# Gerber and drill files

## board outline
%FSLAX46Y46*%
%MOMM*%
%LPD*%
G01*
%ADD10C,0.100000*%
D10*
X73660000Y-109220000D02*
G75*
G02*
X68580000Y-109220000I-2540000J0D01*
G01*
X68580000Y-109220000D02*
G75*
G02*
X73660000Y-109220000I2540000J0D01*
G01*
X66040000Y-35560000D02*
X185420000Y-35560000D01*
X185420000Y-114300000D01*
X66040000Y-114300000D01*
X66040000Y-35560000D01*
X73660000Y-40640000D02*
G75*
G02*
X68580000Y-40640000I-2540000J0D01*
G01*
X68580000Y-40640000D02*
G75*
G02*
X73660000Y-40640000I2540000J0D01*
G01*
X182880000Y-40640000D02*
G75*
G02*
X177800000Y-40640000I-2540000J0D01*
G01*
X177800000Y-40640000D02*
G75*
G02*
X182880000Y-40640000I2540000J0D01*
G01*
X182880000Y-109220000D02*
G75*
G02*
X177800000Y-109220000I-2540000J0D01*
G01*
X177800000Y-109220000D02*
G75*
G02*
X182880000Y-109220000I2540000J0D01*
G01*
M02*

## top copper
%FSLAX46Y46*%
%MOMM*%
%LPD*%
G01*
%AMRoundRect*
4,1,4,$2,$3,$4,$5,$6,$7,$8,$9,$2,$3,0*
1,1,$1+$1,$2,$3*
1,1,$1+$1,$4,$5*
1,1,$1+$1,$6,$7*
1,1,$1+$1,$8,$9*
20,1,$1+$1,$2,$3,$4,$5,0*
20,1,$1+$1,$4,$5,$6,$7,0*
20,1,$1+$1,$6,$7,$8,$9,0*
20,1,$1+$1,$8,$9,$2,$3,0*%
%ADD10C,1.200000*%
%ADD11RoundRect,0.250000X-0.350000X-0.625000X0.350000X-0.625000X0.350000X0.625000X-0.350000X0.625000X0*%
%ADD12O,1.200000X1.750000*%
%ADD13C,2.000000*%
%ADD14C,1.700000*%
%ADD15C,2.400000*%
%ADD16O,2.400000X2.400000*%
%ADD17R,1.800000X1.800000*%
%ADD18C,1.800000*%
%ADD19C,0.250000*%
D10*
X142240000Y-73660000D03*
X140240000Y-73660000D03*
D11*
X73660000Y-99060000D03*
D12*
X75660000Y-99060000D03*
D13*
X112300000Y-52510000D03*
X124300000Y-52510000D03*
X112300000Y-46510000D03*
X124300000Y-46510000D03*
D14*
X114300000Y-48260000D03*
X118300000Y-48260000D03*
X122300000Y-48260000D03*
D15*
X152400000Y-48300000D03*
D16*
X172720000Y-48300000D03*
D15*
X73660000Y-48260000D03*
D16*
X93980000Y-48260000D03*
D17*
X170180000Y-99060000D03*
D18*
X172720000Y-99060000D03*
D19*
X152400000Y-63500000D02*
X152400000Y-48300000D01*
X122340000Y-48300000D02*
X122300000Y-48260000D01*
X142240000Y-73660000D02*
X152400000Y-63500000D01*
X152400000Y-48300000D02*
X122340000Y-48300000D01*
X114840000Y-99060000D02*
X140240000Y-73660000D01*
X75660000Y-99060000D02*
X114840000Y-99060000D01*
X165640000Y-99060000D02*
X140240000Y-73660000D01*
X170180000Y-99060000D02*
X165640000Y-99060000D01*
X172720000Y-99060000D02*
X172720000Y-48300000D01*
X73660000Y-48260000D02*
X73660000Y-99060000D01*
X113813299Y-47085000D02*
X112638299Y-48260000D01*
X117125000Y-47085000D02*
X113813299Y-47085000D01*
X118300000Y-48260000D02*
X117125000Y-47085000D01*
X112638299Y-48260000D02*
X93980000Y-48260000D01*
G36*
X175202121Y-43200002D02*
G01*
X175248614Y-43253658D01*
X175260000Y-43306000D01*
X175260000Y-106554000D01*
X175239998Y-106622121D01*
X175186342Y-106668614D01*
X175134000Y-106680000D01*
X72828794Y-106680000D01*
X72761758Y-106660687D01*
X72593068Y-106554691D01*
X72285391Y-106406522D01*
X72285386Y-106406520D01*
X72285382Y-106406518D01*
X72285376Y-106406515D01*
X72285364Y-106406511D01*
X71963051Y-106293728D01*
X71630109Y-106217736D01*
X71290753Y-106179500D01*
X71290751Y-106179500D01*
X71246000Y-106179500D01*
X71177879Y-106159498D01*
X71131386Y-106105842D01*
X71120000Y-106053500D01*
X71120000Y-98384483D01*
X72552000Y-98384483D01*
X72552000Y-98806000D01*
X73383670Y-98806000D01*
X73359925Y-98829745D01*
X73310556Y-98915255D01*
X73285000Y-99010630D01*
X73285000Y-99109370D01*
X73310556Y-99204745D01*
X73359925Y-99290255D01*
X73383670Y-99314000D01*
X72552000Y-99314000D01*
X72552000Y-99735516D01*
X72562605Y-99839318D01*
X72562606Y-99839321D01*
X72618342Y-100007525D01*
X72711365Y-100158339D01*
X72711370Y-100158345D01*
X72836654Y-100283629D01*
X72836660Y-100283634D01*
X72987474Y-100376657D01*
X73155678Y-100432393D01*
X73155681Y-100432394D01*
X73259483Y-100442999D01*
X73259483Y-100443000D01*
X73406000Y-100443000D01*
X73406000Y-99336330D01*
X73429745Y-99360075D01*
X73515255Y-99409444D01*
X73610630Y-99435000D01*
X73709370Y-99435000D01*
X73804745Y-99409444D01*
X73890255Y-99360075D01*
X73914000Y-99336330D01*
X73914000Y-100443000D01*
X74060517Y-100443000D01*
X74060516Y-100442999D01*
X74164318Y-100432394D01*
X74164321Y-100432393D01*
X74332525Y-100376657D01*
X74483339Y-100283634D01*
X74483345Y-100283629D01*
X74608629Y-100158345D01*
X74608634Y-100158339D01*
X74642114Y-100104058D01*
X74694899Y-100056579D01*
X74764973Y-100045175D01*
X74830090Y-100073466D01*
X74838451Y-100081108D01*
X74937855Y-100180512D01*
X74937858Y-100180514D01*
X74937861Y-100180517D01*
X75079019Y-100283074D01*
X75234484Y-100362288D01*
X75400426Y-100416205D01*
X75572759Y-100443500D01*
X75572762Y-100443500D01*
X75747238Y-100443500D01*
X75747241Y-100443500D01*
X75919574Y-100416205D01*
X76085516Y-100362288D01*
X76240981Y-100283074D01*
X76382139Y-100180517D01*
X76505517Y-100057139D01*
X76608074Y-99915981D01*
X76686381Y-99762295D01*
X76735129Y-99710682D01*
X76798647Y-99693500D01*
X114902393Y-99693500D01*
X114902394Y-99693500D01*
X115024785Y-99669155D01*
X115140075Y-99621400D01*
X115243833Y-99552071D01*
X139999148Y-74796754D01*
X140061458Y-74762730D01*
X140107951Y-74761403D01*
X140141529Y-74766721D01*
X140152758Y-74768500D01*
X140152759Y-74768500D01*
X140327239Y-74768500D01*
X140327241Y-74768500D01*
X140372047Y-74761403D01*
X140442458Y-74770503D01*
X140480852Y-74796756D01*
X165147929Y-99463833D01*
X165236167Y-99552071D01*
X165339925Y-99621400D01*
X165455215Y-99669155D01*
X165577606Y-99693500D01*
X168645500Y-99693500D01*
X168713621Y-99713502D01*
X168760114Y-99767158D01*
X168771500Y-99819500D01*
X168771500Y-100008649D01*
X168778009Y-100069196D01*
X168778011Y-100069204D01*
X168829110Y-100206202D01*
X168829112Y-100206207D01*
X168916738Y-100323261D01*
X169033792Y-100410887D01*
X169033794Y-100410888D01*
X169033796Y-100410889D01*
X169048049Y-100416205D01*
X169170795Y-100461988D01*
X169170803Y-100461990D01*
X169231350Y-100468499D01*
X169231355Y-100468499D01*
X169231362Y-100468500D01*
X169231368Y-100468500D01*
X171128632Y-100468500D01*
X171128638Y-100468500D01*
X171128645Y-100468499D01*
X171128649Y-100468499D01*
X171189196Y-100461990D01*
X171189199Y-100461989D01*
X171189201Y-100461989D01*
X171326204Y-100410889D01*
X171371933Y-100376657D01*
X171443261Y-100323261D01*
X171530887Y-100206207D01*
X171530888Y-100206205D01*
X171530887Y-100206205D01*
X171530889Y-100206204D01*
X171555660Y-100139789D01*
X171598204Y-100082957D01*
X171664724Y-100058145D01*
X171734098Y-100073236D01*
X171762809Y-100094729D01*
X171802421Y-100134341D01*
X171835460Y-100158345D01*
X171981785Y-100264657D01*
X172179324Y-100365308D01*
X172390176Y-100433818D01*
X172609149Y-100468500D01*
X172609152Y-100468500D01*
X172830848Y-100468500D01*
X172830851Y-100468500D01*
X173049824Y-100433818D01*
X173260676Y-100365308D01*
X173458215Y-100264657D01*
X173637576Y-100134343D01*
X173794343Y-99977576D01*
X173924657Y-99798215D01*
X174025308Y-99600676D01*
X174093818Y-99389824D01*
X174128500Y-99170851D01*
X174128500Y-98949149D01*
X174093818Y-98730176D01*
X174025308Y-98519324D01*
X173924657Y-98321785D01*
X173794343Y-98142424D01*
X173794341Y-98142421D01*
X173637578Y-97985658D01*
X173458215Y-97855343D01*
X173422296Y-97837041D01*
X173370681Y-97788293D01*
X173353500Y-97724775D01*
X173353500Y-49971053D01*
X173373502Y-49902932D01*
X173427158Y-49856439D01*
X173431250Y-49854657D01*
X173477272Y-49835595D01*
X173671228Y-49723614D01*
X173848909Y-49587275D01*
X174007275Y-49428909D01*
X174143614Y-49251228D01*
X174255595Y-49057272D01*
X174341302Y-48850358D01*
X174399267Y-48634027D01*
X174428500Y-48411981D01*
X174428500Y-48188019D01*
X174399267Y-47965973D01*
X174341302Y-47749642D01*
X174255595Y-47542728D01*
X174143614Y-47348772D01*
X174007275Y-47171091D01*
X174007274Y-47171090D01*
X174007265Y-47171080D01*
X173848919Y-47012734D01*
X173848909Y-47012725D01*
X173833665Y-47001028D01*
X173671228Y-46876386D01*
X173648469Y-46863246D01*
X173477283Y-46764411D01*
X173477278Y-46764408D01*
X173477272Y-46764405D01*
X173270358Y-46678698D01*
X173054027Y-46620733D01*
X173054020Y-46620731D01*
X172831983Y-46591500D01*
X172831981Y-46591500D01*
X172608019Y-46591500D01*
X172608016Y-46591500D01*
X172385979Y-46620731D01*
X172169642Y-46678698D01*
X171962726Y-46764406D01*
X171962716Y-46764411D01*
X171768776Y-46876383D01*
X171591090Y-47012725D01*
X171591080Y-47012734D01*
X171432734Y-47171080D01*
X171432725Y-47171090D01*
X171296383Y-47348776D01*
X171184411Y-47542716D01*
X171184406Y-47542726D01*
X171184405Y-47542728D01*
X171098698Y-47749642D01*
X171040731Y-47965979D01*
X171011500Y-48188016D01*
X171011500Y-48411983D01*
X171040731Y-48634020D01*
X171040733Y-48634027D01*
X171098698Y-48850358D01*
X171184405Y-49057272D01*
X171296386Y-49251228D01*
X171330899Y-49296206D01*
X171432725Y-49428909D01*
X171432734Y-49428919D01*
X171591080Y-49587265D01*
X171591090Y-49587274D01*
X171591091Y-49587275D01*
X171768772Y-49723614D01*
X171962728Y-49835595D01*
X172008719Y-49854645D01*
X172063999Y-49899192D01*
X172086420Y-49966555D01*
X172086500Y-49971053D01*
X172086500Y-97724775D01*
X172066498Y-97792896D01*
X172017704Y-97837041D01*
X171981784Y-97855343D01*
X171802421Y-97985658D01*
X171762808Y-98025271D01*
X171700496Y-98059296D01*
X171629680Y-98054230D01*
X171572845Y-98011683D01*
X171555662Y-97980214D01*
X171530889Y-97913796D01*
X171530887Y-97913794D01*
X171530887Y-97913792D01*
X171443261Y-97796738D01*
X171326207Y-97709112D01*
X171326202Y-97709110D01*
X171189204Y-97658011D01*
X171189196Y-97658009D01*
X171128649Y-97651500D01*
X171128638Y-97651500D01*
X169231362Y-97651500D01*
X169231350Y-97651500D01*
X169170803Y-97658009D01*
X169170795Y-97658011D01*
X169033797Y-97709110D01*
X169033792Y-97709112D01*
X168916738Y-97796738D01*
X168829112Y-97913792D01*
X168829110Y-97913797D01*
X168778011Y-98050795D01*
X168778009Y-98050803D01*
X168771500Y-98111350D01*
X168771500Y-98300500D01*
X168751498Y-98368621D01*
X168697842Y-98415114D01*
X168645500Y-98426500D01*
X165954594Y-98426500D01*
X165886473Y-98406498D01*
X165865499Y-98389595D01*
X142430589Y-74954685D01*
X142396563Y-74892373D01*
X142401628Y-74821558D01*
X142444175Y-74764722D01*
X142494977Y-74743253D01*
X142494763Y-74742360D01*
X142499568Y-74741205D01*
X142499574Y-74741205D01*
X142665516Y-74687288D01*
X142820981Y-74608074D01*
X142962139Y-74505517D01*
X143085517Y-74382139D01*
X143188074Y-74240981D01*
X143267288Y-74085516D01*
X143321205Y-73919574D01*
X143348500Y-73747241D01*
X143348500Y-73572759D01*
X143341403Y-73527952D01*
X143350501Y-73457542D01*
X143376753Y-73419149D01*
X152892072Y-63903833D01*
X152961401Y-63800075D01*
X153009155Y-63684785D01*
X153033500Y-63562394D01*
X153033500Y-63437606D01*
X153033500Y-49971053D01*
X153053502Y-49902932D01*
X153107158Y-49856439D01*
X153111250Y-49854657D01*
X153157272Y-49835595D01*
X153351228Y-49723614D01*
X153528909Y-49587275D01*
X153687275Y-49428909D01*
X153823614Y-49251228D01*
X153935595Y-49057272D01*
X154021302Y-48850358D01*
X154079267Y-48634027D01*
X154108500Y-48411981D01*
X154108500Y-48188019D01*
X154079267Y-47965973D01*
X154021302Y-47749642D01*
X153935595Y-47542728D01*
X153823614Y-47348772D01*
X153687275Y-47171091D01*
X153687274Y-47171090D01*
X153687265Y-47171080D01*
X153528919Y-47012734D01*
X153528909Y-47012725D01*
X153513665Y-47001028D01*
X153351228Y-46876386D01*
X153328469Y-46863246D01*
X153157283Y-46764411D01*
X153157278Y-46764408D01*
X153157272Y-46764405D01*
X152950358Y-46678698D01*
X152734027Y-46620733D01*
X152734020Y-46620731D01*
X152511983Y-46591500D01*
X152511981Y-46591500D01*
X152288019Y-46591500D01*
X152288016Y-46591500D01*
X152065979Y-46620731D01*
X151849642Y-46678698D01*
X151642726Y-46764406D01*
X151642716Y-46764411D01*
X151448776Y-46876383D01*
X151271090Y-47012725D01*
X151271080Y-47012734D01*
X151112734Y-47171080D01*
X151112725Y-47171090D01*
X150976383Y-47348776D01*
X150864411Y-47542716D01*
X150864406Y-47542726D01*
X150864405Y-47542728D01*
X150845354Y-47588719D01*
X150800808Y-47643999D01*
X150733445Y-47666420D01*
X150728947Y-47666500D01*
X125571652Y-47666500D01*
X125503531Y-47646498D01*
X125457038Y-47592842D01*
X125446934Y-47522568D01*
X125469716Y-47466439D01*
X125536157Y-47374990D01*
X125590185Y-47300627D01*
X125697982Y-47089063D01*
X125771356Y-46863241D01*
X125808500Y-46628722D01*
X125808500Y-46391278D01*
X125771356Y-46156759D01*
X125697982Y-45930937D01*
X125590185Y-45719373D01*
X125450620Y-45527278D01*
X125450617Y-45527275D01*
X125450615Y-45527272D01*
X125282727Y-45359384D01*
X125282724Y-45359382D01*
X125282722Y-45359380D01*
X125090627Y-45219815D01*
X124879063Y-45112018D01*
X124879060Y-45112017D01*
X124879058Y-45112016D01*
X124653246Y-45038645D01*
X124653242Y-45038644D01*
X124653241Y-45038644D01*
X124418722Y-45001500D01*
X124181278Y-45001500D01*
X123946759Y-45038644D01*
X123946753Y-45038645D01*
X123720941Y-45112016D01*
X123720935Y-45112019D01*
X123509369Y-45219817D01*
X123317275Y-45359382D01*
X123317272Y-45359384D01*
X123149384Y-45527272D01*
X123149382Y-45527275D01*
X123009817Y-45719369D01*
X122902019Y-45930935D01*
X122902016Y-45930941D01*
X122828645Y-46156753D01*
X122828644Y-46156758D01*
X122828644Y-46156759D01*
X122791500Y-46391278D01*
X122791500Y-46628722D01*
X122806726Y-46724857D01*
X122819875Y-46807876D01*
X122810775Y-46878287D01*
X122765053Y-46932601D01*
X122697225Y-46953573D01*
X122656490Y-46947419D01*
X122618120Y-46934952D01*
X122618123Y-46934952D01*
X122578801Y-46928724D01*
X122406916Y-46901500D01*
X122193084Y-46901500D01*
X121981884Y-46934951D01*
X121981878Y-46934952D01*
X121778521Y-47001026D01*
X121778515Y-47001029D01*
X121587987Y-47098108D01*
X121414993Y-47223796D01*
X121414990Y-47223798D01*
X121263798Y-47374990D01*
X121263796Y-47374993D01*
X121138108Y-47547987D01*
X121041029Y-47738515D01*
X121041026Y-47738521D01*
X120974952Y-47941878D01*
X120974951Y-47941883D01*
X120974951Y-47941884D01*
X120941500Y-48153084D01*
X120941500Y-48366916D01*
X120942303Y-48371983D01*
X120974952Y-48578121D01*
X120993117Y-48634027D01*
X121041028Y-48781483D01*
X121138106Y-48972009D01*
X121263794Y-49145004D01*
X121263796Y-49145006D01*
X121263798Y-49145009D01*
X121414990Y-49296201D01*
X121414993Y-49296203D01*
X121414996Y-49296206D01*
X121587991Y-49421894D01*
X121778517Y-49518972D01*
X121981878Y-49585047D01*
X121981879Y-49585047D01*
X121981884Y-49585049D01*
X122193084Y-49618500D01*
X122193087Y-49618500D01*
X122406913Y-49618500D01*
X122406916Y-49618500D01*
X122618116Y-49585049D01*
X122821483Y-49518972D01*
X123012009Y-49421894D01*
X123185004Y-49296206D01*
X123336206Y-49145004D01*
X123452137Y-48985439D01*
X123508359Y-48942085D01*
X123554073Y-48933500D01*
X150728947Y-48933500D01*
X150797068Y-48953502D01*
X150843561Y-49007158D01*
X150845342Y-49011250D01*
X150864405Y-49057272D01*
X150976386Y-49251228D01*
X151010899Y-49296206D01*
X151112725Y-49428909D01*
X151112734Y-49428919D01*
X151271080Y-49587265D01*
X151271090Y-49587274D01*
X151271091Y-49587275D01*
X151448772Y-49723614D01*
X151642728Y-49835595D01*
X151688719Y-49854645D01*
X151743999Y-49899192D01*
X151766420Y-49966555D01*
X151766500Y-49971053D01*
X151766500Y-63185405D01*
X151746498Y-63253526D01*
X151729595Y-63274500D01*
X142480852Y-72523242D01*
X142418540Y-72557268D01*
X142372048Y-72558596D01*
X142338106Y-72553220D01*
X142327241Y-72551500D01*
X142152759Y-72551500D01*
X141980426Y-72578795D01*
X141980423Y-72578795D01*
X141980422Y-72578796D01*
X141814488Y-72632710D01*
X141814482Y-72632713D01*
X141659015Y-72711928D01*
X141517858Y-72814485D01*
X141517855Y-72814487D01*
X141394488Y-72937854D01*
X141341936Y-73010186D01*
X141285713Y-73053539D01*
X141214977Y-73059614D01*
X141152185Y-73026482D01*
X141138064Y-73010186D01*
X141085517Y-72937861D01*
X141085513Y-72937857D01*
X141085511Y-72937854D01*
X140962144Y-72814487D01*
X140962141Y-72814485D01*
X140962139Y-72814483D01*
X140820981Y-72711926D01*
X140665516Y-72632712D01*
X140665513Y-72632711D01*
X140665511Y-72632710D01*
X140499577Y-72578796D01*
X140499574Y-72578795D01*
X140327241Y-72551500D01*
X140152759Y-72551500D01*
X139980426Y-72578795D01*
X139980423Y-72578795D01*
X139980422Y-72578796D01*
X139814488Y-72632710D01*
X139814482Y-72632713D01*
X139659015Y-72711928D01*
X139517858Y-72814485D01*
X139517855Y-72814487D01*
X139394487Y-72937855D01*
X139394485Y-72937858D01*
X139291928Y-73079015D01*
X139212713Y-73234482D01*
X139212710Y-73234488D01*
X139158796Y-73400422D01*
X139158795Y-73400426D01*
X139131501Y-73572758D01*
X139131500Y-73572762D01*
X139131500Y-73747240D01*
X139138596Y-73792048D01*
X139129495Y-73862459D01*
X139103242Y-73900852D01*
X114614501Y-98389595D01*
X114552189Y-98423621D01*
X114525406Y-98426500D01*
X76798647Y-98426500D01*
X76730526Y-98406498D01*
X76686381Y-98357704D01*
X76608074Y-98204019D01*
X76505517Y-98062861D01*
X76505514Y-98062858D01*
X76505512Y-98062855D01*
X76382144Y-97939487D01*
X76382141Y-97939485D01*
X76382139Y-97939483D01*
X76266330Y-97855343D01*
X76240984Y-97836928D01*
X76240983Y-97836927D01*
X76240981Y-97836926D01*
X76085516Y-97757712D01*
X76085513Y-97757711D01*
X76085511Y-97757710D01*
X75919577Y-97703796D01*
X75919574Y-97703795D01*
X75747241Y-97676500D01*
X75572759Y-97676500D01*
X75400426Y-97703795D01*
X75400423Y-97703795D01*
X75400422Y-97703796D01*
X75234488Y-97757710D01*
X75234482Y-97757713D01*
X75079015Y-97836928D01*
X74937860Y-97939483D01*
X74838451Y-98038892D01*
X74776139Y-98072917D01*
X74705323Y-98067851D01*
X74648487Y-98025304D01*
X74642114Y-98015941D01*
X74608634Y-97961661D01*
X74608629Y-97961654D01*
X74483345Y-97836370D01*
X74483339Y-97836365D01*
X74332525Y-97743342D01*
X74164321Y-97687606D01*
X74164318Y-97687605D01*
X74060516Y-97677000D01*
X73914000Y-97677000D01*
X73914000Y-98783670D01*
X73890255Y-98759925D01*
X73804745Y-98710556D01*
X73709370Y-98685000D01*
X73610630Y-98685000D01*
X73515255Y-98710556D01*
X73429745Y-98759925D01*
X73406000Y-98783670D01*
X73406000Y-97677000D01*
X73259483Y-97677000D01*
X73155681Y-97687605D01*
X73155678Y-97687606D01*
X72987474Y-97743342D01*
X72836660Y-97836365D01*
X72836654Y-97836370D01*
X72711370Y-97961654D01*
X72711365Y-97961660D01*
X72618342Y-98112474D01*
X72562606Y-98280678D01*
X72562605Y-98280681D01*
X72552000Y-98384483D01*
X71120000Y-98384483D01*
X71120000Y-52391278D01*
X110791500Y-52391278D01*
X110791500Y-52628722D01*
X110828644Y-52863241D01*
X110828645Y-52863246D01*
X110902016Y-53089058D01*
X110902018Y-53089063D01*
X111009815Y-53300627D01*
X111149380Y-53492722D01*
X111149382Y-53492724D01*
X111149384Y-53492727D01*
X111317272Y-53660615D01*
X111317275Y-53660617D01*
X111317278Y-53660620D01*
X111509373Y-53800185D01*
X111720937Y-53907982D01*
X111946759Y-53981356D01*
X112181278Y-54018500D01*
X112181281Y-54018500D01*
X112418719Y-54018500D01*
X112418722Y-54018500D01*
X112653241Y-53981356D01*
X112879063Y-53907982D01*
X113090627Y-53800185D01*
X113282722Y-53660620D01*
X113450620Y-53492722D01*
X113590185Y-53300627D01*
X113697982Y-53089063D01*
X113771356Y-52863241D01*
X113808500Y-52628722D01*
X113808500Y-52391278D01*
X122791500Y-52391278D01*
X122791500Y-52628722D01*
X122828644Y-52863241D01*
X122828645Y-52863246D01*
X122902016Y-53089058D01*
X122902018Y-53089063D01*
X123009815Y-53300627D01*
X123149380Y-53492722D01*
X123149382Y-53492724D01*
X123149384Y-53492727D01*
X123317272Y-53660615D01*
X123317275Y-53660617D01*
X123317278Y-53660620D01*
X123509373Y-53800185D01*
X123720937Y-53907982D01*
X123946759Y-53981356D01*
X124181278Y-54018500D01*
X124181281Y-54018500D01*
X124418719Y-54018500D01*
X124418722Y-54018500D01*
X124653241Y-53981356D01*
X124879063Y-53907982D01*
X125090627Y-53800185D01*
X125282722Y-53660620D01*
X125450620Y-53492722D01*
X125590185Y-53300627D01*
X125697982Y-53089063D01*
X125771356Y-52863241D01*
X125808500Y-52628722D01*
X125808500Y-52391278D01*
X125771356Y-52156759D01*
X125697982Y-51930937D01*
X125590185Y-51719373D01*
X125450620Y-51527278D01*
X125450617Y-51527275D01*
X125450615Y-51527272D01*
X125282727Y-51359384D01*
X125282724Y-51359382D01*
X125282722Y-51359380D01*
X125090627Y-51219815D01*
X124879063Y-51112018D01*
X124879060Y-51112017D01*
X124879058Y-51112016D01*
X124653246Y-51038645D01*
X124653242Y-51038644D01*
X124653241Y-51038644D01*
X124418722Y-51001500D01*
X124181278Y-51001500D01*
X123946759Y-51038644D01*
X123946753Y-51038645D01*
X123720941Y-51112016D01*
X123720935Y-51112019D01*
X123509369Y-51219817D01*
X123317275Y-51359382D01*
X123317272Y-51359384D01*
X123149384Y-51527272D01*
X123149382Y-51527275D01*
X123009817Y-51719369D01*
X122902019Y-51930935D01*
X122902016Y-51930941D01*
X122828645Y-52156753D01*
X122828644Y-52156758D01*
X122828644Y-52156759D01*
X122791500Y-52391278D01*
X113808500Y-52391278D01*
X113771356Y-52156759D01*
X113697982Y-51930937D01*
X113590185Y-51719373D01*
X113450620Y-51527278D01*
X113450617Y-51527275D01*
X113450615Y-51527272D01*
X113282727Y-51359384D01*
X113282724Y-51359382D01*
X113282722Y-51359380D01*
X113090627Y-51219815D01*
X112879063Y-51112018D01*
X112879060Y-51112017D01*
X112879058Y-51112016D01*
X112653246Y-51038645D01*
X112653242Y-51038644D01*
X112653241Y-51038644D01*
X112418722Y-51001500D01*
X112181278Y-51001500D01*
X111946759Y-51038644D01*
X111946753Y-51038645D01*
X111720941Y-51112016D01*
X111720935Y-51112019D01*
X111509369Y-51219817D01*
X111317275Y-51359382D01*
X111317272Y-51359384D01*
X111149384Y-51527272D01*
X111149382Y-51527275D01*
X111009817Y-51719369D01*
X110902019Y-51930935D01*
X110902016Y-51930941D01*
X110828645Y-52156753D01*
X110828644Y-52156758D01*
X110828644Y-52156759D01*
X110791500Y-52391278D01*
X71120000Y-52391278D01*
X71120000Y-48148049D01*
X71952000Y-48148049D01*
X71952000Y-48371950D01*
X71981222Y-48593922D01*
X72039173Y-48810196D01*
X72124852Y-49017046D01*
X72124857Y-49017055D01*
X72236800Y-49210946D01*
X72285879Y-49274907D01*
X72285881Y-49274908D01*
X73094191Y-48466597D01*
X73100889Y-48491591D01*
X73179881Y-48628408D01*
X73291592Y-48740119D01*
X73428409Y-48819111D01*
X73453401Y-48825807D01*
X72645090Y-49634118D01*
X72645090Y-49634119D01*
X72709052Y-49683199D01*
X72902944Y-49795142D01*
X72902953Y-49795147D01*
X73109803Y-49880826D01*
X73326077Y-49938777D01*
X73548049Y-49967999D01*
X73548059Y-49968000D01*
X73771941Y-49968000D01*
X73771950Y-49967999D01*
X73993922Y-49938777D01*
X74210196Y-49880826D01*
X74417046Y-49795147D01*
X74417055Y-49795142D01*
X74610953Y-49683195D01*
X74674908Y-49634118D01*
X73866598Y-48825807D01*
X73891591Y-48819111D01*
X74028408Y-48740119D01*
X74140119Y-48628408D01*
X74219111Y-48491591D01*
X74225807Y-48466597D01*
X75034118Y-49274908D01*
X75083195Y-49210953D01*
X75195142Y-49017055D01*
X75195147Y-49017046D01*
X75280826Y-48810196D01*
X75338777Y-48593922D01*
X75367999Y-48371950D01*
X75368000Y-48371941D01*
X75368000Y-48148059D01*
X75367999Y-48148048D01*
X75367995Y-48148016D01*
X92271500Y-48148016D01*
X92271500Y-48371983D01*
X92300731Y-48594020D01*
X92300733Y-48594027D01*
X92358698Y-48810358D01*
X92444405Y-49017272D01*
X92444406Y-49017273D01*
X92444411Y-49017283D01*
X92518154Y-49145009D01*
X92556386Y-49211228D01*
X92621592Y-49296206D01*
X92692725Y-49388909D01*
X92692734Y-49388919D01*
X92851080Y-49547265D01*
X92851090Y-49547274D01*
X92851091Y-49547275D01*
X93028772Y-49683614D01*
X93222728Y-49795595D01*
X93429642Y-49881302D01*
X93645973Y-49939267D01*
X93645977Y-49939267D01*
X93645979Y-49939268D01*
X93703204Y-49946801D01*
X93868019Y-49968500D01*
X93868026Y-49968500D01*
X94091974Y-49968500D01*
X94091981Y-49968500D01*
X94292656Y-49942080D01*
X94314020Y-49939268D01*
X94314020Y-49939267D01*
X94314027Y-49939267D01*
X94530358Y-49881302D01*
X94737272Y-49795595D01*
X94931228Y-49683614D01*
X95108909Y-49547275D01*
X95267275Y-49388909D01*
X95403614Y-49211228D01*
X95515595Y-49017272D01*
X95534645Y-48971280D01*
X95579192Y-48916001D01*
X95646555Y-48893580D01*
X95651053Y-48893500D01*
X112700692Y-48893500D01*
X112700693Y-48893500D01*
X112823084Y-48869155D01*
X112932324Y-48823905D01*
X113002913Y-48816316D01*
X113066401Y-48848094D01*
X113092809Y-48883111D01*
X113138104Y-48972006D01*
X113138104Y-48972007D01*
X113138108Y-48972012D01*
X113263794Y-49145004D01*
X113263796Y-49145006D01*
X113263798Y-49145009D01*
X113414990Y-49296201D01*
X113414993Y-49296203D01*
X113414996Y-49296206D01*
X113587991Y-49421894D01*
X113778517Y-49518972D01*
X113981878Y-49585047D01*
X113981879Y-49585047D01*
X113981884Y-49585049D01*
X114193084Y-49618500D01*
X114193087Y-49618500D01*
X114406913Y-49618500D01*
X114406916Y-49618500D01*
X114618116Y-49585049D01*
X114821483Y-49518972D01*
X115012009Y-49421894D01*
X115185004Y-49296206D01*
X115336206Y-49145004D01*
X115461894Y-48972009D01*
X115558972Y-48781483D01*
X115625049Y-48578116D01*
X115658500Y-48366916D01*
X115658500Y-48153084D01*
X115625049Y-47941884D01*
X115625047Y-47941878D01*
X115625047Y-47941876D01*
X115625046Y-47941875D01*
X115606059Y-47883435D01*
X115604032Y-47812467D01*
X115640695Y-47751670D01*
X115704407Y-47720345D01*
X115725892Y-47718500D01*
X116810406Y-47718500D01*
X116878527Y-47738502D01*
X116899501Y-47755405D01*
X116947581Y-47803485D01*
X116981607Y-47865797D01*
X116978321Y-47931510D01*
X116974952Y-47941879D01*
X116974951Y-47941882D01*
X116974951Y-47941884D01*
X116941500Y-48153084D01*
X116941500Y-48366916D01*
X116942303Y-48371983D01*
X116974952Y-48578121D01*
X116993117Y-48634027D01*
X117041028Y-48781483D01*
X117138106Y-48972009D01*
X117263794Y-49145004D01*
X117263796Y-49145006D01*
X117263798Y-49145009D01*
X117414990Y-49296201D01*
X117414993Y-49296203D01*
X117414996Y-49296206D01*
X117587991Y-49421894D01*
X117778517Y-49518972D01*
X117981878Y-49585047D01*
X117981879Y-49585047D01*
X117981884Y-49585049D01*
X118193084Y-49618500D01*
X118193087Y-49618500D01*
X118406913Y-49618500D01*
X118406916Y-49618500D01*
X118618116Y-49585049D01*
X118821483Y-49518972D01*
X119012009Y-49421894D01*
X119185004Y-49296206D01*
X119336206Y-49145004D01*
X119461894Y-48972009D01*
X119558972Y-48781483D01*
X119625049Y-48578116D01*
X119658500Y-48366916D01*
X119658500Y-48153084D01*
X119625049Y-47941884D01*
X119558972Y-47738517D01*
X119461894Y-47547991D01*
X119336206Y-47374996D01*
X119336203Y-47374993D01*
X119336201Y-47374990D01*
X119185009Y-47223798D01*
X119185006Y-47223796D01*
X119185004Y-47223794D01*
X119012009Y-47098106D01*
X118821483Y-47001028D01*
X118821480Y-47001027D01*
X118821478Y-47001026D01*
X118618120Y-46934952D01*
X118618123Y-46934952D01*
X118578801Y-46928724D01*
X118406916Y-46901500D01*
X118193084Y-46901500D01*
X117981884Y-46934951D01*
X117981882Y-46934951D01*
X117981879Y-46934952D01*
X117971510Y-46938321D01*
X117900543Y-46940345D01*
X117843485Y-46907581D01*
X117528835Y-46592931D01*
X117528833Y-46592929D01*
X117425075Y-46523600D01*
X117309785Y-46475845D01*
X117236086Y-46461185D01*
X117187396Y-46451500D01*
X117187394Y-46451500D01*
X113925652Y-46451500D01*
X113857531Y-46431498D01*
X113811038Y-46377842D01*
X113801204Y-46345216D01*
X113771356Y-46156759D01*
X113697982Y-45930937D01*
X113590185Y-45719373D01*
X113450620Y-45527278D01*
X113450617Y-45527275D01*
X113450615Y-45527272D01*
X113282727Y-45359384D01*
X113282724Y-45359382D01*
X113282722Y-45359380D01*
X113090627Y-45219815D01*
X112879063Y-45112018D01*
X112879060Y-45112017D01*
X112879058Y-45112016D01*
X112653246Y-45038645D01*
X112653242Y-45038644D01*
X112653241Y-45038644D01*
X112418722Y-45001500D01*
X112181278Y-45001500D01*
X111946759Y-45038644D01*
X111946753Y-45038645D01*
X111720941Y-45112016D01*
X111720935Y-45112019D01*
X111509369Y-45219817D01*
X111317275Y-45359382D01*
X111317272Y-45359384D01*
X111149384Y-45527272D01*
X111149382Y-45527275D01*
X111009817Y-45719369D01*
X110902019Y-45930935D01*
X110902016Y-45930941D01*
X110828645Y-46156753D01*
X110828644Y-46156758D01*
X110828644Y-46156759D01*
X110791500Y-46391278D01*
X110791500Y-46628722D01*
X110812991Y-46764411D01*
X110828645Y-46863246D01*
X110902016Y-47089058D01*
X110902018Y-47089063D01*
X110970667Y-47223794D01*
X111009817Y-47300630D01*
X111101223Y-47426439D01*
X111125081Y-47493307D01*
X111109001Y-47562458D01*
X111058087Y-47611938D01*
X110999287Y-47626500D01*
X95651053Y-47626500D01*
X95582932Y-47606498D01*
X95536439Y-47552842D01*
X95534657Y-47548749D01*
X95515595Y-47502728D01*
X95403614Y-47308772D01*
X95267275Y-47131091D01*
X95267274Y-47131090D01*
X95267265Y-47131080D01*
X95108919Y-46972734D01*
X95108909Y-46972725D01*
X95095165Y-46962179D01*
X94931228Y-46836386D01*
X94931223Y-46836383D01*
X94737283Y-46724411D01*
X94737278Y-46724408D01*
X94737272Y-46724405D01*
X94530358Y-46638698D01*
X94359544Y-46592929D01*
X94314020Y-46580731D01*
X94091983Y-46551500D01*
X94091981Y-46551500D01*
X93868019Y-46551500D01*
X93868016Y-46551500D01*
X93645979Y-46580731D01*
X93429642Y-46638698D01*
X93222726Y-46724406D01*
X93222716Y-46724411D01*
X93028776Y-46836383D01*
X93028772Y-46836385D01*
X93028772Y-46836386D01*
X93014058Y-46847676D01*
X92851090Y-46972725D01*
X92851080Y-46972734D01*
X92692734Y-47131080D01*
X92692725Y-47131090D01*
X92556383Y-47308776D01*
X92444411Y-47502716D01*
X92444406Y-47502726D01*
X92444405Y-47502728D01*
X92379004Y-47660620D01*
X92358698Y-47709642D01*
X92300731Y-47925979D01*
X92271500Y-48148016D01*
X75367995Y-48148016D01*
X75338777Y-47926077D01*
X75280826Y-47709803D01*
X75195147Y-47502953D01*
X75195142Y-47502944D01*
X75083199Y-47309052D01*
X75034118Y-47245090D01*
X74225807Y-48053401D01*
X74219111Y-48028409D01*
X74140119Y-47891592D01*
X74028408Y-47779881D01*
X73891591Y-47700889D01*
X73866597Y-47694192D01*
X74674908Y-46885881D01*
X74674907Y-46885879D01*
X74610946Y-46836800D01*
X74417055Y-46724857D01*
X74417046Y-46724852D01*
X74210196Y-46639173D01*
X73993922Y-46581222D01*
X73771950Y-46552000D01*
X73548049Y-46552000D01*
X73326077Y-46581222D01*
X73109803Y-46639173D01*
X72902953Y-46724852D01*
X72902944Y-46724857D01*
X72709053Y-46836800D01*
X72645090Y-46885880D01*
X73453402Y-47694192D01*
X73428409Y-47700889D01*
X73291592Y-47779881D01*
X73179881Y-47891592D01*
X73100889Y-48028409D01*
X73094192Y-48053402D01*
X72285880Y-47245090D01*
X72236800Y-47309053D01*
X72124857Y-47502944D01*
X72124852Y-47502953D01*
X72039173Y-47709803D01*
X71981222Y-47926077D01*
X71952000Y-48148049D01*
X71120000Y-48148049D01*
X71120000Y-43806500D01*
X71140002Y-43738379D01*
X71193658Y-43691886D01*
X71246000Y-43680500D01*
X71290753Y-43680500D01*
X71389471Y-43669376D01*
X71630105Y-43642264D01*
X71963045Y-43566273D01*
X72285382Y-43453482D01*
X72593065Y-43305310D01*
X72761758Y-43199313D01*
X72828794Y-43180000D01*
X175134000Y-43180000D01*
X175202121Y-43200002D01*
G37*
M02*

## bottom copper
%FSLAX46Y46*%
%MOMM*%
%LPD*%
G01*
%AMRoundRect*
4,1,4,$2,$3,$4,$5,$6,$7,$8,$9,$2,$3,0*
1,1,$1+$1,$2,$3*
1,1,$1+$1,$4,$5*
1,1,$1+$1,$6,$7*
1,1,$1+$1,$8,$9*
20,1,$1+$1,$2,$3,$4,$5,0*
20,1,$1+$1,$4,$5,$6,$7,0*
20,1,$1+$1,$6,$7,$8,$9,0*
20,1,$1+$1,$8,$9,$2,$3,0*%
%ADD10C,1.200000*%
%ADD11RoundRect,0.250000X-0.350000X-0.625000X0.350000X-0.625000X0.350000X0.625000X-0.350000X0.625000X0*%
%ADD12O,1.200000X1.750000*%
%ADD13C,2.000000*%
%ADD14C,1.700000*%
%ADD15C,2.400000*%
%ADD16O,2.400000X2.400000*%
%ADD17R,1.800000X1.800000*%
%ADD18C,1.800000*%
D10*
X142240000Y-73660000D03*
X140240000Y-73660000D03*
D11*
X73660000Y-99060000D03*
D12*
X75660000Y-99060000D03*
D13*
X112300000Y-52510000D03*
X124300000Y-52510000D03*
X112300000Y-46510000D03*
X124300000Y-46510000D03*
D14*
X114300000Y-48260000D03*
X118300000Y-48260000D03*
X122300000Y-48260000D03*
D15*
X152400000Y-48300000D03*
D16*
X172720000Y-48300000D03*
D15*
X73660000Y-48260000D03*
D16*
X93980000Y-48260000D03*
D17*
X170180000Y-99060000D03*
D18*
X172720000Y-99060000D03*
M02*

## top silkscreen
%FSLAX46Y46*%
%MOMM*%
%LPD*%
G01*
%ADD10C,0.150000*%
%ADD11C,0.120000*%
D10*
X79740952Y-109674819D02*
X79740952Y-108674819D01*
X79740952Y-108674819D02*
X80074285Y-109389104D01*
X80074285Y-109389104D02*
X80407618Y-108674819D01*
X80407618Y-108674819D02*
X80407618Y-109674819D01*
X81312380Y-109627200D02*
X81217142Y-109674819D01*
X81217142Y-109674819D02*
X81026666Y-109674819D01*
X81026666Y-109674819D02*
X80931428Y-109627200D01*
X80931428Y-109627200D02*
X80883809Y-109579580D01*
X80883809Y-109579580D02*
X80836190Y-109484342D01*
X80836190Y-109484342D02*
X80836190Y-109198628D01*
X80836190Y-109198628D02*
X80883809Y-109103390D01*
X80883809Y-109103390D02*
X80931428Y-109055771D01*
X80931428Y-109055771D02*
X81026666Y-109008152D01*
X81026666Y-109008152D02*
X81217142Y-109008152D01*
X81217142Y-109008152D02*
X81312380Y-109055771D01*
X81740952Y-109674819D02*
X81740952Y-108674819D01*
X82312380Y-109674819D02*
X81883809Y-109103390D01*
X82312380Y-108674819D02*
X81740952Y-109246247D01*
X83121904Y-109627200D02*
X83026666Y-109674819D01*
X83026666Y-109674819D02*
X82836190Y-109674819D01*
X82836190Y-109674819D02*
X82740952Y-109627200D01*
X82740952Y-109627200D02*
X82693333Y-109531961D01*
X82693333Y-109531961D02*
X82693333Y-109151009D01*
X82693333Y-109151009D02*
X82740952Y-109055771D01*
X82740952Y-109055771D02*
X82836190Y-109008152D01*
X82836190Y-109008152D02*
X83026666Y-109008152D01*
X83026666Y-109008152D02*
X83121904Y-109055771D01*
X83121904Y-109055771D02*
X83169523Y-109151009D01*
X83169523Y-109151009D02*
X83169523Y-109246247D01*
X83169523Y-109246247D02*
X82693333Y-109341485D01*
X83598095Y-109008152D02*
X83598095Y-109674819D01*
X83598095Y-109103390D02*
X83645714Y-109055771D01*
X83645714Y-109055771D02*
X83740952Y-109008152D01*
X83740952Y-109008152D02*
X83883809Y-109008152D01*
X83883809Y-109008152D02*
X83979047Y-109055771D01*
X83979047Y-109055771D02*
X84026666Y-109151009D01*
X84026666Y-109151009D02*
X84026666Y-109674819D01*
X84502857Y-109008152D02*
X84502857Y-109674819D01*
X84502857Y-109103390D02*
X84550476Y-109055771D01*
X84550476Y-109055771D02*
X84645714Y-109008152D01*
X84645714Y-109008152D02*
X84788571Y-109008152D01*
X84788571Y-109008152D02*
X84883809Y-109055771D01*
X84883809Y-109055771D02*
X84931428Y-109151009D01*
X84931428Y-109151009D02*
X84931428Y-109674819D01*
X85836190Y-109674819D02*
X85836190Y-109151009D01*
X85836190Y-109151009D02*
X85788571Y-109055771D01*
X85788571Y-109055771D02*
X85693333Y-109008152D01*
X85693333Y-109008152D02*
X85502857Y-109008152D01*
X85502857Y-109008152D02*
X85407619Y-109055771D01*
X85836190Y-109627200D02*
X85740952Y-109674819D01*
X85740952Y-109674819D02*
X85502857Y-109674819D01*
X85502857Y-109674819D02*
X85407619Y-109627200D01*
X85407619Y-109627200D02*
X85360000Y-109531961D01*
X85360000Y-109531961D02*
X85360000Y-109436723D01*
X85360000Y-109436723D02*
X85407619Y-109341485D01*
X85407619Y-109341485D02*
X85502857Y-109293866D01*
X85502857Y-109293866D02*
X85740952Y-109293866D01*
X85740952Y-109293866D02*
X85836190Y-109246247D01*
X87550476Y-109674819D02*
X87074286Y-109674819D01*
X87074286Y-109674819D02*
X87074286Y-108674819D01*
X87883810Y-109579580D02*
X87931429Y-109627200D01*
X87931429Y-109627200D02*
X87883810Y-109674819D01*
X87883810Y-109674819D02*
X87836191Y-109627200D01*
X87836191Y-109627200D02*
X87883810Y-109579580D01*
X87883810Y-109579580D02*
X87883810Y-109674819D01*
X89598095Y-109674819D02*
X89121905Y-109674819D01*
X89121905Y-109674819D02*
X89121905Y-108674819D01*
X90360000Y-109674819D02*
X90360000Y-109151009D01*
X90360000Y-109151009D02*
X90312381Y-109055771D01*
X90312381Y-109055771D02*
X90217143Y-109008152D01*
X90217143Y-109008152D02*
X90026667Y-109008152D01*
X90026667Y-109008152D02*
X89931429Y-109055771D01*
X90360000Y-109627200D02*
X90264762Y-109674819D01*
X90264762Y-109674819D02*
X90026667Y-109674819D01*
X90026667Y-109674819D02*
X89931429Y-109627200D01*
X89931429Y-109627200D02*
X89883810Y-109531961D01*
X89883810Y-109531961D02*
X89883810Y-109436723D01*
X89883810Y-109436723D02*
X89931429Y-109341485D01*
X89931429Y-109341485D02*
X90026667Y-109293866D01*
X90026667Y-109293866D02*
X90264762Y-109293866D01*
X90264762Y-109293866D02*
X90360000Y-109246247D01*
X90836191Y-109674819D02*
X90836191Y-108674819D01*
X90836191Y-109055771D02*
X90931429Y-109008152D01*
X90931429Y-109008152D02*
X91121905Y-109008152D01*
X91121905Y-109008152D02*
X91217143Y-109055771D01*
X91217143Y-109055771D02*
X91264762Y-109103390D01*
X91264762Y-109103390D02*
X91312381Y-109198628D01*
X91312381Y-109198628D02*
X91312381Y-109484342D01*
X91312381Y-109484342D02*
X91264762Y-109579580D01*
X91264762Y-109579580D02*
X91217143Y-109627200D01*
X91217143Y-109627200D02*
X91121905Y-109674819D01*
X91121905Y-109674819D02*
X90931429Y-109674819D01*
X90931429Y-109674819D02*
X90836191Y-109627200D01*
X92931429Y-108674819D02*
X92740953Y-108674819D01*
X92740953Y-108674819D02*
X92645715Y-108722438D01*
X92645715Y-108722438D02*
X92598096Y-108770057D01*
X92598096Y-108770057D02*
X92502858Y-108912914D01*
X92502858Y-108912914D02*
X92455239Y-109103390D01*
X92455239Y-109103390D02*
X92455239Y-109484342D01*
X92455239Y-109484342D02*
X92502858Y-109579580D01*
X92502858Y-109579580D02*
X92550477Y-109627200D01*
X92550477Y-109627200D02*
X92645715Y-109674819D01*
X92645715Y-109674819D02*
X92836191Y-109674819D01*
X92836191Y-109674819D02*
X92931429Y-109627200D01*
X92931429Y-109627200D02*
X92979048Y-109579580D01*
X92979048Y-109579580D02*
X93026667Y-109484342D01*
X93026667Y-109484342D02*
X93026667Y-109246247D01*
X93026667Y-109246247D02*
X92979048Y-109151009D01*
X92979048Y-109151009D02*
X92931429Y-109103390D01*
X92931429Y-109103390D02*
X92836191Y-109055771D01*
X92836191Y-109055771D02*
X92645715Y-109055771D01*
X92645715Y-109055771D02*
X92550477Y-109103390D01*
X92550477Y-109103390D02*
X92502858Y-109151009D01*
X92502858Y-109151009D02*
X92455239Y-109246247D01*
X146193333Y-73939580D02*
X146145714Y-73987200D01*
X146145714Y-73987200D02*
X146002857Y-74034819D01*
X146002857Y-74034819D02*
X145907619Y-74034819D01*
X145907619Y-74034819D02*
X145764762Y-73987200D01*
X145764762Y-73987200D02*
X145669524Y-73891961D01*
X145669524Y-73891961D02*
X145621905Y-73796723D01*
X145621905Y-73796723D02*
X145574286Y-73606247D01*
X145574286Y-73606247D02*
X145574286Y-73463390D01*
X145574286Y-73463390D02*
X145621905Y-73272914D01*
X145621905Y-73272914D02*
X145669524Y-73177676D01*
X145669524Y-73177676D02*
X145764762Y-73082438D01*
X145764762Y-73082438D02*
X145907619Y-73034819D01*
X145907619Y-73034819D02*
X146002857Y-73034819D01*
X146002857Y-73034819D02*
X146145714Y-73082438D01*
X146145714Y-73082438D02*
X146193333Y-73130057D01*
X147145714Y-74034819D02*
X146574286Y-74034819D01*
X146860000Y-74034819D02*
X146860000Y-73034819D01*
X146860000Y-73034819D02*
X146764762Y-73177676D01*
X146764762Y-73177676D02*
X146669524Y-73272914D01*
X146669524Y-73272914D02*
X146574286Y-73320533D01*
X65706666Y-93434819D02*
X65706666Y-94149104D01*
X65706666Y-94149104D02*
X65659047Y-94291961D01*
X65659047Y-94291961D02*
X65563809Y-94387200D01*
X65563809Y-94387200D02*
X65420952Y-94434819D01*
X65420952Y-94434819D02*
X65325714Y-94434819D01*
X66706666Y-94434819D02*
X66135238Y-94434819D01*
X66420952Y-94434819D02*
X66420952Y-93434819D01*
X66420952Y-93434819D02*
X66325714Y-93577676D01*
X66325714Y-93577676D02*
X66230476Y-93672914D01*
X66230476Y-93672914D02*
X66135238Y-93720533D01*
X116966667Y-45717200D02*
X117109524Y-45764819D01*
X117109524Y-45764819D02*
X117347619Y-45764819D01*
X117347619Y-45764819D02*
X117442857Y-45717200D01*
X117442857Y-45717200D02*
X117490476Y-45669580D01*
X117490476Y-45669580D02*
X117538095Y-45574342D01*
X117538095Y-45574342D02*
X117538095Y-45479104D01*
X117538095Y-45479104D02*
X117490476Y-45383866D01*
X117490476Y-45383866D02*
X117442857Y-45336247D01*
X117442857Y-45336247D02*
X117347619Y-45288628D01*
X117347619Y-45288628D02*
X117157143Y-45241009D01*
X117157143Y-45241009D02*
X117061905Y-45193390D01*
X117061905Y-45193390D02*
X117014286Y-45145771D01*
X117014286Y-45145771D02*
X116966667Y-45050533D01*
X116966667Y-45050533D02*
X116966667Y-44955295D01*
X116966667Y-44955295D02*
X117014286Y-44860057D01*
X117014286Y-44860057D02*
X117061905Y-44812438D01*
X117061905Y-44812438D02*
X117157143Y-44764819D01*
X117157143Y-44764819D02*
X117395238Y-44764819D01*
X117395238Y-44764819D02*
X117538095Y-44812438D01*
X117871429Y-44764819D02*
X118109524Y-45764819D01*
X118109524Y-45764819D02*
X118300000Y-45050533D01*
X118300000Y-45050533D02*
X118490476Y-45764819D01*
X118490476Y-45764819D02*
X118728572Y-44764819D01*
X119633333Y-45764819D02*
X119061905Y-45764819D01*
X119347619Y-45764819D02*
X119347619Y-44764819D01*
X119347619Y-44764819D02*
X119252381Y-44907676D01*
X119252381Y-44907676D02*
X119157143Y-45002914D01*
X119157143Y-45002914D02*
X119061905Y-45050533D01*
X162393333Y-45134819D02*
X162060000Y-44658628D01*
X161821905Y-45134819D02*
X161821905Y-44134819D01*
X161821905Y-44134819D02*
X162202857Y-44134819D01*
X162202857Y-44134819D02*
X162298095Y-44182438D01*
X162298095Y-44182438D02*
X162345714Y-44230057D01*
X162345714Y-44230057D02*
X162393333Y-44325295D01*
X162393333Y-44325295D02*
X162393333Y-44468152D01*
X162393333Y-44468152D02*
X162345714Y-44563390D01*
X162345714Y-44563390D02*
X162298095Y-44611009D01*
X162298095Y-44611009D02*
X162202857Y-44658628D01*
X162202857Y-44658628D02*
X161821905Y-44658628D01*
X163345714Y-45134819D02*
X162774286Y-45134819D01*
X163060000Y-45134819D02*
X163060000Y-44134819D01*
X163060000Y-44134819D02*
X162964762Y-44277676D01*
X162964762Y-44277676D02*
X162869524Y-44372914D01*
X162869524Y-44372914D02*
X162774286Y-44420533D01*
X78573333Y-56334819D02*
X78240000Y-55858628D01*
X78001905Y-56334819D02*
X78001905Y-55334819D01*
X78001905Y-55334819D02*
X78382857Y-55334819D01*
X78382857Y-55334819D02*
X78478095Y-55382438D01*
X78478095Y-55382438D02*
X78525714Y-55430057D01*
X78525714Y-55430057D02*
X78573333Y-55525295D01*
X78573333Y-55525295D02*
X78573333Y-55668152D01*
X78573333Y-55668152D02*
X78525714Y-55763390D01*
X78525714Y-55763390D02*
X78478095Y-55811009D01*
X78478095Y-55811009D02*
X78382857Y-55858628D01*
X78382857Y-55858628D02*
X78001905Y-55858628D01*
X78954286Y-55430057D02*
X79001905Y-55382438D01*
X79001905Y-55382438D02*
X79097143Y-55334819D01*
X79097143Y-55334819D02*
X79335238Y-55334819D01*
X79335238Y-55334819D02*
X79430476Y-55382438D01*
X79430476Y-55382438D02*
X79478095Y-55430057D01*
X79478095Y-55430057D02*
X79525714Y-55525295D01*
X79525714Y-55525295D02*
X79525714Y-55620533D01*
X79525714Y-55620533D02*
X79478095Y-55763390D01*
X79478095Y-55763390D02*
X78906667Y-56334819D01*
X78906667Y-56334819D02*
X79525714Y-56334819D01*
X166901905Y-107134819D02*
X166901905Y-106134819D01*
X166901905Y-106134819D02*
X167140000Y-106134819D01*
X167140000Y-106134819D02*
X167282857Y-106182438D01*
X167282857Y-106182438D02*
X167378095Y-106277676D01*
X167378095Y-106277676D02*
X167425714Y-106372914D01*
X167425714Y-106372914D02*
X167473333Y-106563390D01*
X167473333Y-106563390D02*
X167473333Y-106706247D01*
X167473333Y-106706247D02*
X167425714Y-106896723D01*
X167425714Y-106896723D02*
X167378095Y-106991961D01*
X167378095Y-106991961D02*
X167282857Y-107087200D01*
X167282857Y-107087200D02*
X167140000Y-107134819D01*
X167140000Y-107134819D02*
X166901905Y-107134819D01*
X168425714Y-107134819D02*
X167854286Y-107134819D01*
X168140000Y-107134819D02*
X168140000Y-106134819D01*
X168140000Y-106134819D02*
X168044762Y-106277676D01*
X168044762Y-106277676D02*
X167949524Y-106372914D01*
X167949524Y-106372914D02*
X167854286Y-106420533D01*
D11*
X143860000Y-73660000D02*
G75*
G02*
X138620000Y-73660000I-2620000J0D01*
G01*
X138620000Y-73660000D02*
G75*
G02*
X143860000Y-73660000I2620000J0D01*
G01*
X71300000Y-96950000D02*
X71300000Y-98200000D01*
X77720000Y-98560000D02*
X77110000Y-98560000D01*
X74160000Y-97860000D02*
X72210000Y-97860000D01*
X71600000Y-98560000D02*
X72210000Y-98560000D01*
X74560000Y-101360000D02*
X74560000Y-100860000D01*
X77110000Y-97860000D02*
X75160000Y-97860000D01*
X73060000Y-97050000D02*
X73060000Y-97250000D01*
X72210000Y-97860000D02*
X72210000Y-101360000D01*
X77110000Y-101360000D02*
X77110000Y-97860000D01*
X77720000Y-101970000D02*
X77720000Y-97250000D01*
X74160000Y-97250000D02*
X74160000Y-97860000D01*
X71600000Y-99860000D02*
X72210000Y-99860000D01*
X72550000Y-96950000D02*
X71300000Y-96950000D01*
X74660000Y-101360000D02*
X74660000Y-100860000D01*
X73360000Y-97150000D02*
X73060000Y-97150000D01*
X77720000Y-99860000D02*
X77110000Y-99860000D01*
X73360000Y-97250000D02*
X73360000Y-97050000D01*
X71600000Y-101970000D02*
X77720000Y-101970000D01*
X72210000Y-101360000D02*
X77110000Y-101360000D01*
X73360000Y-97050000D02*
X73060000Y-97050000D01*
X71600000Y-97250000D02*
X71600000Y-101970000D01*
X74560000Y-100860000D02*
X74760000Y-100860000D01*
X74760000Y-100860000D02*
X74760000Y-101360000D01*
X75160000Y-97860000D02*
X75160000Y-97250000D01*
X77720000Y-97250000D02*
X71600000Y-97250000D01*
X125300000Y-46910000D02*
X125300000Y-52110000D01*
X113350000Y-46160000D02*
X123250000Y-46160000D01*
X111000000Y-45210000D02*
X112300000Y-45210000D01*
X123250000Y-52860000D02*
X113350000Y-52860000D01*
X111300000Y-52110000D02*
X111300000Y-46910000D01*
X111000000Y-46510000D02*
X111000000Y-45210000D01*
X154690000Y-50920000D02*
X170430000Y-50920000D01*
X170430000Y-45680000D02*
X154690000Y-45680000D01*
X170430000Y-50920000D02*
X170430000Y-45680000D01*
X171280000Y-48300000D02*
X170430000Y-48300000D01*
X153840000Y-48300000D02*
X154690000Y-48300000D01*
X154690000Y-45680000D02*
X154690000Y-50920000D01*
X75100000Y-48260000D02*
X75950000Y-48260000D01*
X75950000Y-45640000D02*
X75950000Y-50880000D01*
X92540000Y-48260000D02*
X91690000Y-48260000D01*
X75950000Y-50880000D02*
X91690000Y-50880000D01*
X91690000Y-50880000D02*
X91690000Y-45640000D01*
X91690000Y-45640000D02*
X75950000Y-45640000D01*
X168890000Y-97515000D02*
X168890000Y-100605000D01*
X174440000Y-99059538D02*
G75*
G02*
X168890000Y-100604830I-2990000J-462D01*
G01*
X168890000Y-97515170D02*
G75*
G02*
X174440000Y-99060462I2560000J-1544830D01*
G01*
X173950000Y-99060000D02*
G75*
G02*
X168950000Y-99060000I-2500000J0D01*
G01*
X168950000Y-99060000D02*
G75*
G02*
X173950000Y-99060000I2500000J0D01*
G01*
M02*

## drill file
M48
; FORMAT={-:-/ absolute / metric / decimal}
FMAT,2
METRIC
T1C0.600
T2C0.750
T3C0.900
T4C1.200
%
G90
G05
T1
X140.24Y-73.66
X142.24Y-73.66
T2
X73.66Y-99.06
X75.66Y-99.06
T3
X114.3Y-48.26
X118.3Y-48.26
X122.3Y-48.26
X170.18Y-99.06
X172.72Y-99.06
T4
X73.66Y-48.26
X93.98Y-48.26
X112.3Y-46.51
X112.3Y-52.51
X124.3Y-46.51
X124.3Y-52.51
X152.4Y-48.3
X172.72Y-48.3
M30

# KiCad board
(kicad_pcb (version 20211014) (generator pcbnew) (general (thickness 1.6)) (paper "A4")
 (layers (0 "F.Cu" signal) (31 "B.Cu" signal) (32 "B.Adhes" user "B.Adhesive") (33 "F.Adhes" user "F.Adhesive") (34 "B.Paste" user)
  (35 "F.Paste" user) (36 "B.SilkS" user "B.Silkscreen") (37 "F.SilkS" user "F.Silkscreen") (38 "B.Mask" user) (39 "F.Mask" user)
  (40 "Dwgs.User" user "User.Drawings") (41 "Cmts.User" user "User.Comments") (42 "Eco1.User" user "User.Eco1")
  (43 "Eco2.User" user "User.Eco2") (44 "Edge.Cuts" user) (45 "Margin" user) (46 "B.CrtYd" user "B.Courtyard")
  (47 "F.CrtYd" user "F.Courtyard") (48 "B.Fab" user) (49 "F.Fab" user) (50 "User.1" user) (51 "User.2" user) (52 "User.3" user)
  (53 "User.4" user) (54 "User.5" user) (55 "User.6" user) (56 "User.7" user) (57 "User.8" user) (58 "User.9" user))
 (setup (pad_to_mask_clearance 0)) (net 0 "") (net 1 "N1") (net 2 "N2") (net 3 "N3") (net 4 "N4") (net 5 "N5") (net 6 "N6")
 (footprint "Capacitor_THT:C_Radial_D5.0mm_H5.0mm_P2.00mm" (layer "F.Cu") (at 142.24 73.66 180)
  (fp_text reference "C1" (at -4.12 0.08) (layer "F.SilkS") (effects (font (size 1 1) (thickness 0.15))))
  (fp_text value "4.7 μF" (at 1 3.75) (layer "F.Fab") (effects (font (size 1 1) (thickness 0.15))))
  (fp_circle (center 1 0) (end 3.62 0) (layer "F.SilkS") (width 0.12) (fill none))
  (pad "1" thru_hole circle (at 0 0 180) (size 1.2 1.2) (drill 0.6) (layers *.Cu *.Mask) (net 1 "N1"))
  (pad "2" thru_hole circle (at 2 0 180) (size 1.2 1.2) (drill 0.6) (layers *.Cu *.Mask) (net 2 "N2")))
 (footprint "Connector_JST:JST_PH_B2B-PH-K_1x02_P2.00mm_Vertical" (layer "F.Cu") (at 73.66 99.06)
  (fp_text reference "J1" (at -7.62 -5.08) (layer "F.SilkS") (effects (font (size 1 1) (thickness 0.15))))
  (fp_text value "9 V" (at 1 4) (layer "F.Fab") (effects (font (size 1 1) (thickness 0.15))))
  (fp_line (start -2.36 -2.11) (end -2.36 -0.86) (layer "F.SilkS") (width 0.12))
  (fp_line (start 4.06 -0.5) (end 3.45 -0.5) (layer "F.SilkS") (width 0.12))
  (fp_line (start 0.5 -1.2) (end -1.45 -1.2) (layer "F.SilkS") (width 0.12))
  (fp_line (start -2.06 -0.5) (end -1.45 -0.5) (layer "F.SilkS") (width 0.12))
  (fp_line (start 0.9 2.3) (end 0.9 1.8) (layer "F.SilkS") (width 0.12))
  (fp_line (start 3.45 -1.2) (end 1.5 -1.2) (layer "F.SilkS") (width 0.12))
  (fp_line (start -0.6 -2.01) (end -0.6 -1.81) (layer "F.SilkS") (width 0.12))
  (fp_line (start -1.45 -1.2) (end -1.45 2.3) (layer "F.SilkS") (width 0.12))
  (fp_line (start 3.45 2.3) (end 3.45 -1.2) (layer "F.SilkS") (width 0.12))
  (fp_line (start 4.06 2.91) (end 4.06 -1.81) (layer "F.SilkS") (width 0.12))
  (fp_line (start 0.5 -1.81) (end 0.5 -1.2) (layer "F.SilkS") (width 0.12))
  (fp_line (start -2.06 0.8) (end -1.45 0.8) (layer "F.SilkS") (width 0.12))
  (fp_line (start -1.11 -2.11) (end -2.36 -2.11) (layer "F.SilkS") (width 0.12))
  (fp_line (start 1 2.3) (end 1 1.8) (layer "F.SilkS") (width 0.12))
  (fp_line (start -0.3 -1.91) (end -0.6 -1.91) (layer "F.SilkS") (width 0.12))
  (fp_line (start 4.06 0.8) (end 3.45 0.8) (layer "F.SilkS") (width 0.12))
  (fp_line (start -0.3 -1.81) (end -0.3 -2.01) (layer "F.SilkS") (width 0.12))
  (fp_line (start -2.06 2.91) (end 4.06 2.91) (layer "F.SilkS") (width 0.12))
  (fp_line (start -1.45 2.3) (end 3.45 2.3) (layer "F.SilkS") (width 0.12))
  (fp_line (start -0.3 -2.01) (end -0.6 -2.01) (layer "F.SilkS") (width 0.12))
  (fp_line (start -2.06 -1.81) (end -2.06 2.91) (layer "F.SilkS") (width 0.12))
  (fp_line (start 0.9 1.8) (end 1.1 1.8) (layer "F.SilkS") (width 0.12))
  (fp_line (start 1.1 1.8) (end 1.1 2.3) (layer "F.SilkS") (width 0.12))
  (fp_line (start 1.5 -1.2) (end 1.5 -1.81) (layer "F.SilkS") (width 0.12))
  (fp_line (start 4.06 -1.81) (end -2.06 -1.81) (layer "F.SilkS") (width 0.12))
  (pad "1" thru_hole roundrect (at 0 0) (size 1.2 1.75) (drill 0.75) (layers *.Cu *.Mask) (roundrect_rratio 0.2083333333) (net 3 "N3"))
  (pad "2" thru_hole oval (at 2 0) (size 1.2 1.75) (drill 0.75) (layers *.Cu *.Mask) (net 2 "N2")))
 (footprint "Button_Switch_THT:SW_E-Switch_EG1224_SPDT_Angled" (layer "F.Cu") (at 114.3 48.26)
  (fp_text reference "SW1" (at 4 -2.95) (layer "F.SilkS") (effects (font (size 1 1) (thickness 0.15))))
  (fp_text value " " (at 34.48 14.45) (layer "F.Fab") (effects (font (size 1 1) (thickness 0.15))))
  (fp_line (start 11 -1.35) (end 11 3.85) (layer "F.SilkS") (width 0.12))
  (fp_line (start -0.95 -2.1) (end 8.95 -2.1) (layer "F.SilkS") (width 0.12))
  (fp_line (start -3.3 -3.05) (end -2 -3.05) (layer "F.SilkS") (width 0.12))
  (fp_line (start 8.95 4.6) (end -0.95 4.6) (layer "F.SilkS") (width 0.12))
  (fp_line (start -3 3.85) (end -3 -1.35) (layer "F.SilkS") (width 0.12))
  (fp_line (start -3.3 -1.75) (end -3.3 -3.05) (layer "F.SilkS") (width 0.12))
  (pad "" thru_hole circle (at -2 4.25) (size 2 2) (drill 1.2) (layers *.Cu *.Mask))
  (pad "" thru_hole circle (at 10 4.25) (size 2 2) (drill 1.2) (layers *.Cu *.Mask))
  (pad "" thru_hole circle (at -2 -1.75) (size 2 2) (drill 1.2) (layers *.Cu *.Mask))
  (pad "" thru_hole circle (at 10 -1.75) (size 2 2) (drill 1.2) (layers *.Cu *.Mask))
  (pad "1" thru_hole circle (at 0 0) (size 1.7 1.7) (drill 0.9) (layers *.Cu *.Mask) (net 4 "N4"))
  (pad "2" thru_hole circle (at 4 0) (size 1.7 1.7) (drill 0.9) (layers *.Cu *.Mask) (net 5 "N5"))
  (pad "3" thru_hole circle (at 8 0) (size 1.7 1.7) (drill 0.9) (layers *.Cu *.Mask) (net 1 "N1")))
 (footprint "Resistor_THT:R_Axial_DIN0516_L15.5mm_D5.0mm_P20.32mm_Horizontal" (layer "F.Cu") (at 152.4 48.3)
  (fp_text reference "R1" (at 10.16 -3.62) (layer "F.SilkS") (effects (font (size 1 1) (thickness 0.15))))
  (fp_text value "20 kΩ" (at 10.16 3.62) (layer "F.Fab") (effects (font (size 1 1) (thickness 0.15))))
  (fp_line (start 2.29 2.62) (end 18.03 2.62) (layer "F.SilkS") (width 0.12))
  (fp_line (start 18.03 -2.62) (end 2.29 -2.62) (layer "F.SilkS") (width 0.12))
  (fp_line (start 18.03 2.62) (end 18.03 -2.62) (layer "F.SilkS") (width 0.12))
  (fp_line (start 18.88 0) (end 18.03 0) (layer "F.SilkS") (width 0.12))
  (fp_line (start 1.44 0) (end 2.29 0) (layer "F.SilkS") (width 0.12))
  (fp_line (start 2.29 -2.62) (end 2.29 2.62) (layer "F.SilkS") (width 0.12))
  (pad "1" thru_hole circle (at 0 0) (size 2.4 2.4) (drill 1.2) (layers *.Cu *.Mask) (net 1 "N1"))
  (pad "2" thru_hole oval (at 20.32 0) (size 2.4 2.4) (drill 1.2) (layers *.Cu *.Mask) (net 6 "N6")))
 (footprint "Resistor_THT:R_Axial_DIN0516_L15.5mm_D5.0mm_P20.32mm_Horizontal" (layer "F.Cu") (at 73.66 48.26)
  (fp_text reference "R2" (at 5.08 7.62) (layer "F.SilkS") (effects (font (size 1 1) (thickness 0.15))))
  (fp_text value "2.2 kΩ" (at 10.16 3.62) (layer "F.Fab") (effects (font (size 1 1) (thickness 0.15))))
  (fp_line (start 1.44 0) (end 2.29 0) (layer "F.SilkS") (width 0.12))
  (fp_line (start 2.29 -2.62) (end 2.29 2.62) (layer "F.SilkS") (width 0.12))
  (fp_line (start 18.88 0) (end 18.03 0) (layer "F.SilkS") (width 0.12))
  (fp_line (start 2.29 2.62) (end 18.03 2.62) (layer "F.SilkS") (width 0.12))
  (fp_line (start 18.03 2.62) (end 18.03 -2.62) (layer "F.SilkS") (width 0.12))
  (fp_line (start 18.03 -2.62) (end 2.29 -2.62) (layer "F.SilkS") (width 0.12))
  (pad "1" thru_hole circle (at 0 0) (size 2.4 2.4) (drill 1.2) (layers *.Cu *.Mask) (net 3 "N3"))
  (pad "2" thru_hole oval (at 20.32 0) (size 2.4 2.4) (drill 1.2) (layers *.Cu *.Mask) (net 5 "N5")))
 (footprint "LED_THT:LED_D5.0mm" (layer "F.Cu") (at 170.18 99.06)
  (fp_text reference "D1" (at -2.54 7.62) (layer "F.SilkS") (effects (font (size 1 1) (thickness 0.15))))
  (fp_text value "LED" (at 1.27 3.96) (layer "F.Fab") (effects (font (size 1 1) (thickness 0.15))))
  (fp_line (start -1.29 -1.545) (end -1.29 1.545) (layer "F.SilkS") (width 0.12))
  (fp_arc (start 4.26 -0.000462) (mid 2.072002 2.880433) (end -1.29 1.54483) (layer "F.SilkS") (width 0.12))
  (fp_arc (start -1.29 -1.54483) (mid 2.072002 -2.880433) (end 4.26 0.000462) (layer "F.SilkS") (width 0.12))
  (fp_circle (center 1.27 0) (end 3.77 0) (layer "F.SilkS") (width 0.12) (fill none))
  (pad "1" thru_hole rect (at 0 0) (size 1.8 1.8) (drill 0.9) (layers *.Cu *.Mask) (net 2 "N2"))
  (pad "2" thru_hole circle (at 2.54 0) (size 1.8 1.8) (drill 0.9) (layers *.Cu *.Mask) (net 6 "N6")))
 (gr_circle (center 71.12 109.22) (end 73.66 109.22) (layer "Edge.Cuts") (width 0.1) (fill none))
 (gr_rect (start 66.04 35.56) (end 185.42 114.3) (layer "Edge.Cuts") (width 0.1) (fill none))
 (gr_circle (center 71.12 40.64) (end 73.66 40.64) (layer "Edge.Cuts") (width 0.1) (fill none))
 (gr_circle (center 180.34 40.64) (end 182.88 40.64) (layer "Edge.Cuts") (width 0.1) (fill none))
 (gr_circle (center 180.34 109.22) (end 180.34 106.68) (layer "Edge.Cuts") (width 0.1) (fill none))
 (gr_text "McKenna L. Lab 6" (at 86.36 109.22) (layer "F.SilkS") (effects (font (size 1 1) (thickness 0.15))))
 (segment (start 152.4 63.5) (end 152.4 48.3) (width 0.25) (layer "F.Cu") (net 1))
 (segment (start 122.34 48.3) (end 122.3 48.26) (width 0.25) (layer "F.Cu") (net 1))
 (segment (start 142.24 73.66) (end 152.4 63.5) (width 0.25) (layer "F.Cu") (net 1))
 (segment (start 152.4 48.3) (end 122.34 48.3) (width 0.25) (layer "F.Cu") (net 1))
 (segment (start 114.84 99.06) (end 140.24 73.66) (width 0.25) (layer "F.Cu") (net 2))
 (segment (start 75.66 99.06) (end 114.84 99.06) (width 0.25) (layer "F.Cu") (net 2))
 (segment (start 165.64 99.06) (end 140.24 73.66) (width 0.25) (layer "F.Cu") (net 2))
 (segment (start 170.18 99.06) (end 165.64 99.06) (width 0.25) (layer "F.Cu") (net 2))
 (segment (start 172.72 99.06) (end 172.72 48.3) (width 0.25) (layer "F.Cu") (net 6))
 (segment (start 73.66 48.26) (end 73.66 99.06) (width 0.25) (layer "F.Cu") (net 3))
 (segment (start 113.813299 47.085) (end 112.638299 48.26) (width 0.25) (layer "F.Cu") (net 5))
 (segment (start 117.125 47.085) (end 113.813299 47.085) (width 0.25) (layer "F.Cu") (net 5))
 (segment (start 118.3 48.26) (end 117.125 47.085) (width 0.25) (layer "F.Cu") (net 5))
 (segment (start 112.638299 48.26) (end 93.98 48.26) (width 0.25) (layer "F.Cu") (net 5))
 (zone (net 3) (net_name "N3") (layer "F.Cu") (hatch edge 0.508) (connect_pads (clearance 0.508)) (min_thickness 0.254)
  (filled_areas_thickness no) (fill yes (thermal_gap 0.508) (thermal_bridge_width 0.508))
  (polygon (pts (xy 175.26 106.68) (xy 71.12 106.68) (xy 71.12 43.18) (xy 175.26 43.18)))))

